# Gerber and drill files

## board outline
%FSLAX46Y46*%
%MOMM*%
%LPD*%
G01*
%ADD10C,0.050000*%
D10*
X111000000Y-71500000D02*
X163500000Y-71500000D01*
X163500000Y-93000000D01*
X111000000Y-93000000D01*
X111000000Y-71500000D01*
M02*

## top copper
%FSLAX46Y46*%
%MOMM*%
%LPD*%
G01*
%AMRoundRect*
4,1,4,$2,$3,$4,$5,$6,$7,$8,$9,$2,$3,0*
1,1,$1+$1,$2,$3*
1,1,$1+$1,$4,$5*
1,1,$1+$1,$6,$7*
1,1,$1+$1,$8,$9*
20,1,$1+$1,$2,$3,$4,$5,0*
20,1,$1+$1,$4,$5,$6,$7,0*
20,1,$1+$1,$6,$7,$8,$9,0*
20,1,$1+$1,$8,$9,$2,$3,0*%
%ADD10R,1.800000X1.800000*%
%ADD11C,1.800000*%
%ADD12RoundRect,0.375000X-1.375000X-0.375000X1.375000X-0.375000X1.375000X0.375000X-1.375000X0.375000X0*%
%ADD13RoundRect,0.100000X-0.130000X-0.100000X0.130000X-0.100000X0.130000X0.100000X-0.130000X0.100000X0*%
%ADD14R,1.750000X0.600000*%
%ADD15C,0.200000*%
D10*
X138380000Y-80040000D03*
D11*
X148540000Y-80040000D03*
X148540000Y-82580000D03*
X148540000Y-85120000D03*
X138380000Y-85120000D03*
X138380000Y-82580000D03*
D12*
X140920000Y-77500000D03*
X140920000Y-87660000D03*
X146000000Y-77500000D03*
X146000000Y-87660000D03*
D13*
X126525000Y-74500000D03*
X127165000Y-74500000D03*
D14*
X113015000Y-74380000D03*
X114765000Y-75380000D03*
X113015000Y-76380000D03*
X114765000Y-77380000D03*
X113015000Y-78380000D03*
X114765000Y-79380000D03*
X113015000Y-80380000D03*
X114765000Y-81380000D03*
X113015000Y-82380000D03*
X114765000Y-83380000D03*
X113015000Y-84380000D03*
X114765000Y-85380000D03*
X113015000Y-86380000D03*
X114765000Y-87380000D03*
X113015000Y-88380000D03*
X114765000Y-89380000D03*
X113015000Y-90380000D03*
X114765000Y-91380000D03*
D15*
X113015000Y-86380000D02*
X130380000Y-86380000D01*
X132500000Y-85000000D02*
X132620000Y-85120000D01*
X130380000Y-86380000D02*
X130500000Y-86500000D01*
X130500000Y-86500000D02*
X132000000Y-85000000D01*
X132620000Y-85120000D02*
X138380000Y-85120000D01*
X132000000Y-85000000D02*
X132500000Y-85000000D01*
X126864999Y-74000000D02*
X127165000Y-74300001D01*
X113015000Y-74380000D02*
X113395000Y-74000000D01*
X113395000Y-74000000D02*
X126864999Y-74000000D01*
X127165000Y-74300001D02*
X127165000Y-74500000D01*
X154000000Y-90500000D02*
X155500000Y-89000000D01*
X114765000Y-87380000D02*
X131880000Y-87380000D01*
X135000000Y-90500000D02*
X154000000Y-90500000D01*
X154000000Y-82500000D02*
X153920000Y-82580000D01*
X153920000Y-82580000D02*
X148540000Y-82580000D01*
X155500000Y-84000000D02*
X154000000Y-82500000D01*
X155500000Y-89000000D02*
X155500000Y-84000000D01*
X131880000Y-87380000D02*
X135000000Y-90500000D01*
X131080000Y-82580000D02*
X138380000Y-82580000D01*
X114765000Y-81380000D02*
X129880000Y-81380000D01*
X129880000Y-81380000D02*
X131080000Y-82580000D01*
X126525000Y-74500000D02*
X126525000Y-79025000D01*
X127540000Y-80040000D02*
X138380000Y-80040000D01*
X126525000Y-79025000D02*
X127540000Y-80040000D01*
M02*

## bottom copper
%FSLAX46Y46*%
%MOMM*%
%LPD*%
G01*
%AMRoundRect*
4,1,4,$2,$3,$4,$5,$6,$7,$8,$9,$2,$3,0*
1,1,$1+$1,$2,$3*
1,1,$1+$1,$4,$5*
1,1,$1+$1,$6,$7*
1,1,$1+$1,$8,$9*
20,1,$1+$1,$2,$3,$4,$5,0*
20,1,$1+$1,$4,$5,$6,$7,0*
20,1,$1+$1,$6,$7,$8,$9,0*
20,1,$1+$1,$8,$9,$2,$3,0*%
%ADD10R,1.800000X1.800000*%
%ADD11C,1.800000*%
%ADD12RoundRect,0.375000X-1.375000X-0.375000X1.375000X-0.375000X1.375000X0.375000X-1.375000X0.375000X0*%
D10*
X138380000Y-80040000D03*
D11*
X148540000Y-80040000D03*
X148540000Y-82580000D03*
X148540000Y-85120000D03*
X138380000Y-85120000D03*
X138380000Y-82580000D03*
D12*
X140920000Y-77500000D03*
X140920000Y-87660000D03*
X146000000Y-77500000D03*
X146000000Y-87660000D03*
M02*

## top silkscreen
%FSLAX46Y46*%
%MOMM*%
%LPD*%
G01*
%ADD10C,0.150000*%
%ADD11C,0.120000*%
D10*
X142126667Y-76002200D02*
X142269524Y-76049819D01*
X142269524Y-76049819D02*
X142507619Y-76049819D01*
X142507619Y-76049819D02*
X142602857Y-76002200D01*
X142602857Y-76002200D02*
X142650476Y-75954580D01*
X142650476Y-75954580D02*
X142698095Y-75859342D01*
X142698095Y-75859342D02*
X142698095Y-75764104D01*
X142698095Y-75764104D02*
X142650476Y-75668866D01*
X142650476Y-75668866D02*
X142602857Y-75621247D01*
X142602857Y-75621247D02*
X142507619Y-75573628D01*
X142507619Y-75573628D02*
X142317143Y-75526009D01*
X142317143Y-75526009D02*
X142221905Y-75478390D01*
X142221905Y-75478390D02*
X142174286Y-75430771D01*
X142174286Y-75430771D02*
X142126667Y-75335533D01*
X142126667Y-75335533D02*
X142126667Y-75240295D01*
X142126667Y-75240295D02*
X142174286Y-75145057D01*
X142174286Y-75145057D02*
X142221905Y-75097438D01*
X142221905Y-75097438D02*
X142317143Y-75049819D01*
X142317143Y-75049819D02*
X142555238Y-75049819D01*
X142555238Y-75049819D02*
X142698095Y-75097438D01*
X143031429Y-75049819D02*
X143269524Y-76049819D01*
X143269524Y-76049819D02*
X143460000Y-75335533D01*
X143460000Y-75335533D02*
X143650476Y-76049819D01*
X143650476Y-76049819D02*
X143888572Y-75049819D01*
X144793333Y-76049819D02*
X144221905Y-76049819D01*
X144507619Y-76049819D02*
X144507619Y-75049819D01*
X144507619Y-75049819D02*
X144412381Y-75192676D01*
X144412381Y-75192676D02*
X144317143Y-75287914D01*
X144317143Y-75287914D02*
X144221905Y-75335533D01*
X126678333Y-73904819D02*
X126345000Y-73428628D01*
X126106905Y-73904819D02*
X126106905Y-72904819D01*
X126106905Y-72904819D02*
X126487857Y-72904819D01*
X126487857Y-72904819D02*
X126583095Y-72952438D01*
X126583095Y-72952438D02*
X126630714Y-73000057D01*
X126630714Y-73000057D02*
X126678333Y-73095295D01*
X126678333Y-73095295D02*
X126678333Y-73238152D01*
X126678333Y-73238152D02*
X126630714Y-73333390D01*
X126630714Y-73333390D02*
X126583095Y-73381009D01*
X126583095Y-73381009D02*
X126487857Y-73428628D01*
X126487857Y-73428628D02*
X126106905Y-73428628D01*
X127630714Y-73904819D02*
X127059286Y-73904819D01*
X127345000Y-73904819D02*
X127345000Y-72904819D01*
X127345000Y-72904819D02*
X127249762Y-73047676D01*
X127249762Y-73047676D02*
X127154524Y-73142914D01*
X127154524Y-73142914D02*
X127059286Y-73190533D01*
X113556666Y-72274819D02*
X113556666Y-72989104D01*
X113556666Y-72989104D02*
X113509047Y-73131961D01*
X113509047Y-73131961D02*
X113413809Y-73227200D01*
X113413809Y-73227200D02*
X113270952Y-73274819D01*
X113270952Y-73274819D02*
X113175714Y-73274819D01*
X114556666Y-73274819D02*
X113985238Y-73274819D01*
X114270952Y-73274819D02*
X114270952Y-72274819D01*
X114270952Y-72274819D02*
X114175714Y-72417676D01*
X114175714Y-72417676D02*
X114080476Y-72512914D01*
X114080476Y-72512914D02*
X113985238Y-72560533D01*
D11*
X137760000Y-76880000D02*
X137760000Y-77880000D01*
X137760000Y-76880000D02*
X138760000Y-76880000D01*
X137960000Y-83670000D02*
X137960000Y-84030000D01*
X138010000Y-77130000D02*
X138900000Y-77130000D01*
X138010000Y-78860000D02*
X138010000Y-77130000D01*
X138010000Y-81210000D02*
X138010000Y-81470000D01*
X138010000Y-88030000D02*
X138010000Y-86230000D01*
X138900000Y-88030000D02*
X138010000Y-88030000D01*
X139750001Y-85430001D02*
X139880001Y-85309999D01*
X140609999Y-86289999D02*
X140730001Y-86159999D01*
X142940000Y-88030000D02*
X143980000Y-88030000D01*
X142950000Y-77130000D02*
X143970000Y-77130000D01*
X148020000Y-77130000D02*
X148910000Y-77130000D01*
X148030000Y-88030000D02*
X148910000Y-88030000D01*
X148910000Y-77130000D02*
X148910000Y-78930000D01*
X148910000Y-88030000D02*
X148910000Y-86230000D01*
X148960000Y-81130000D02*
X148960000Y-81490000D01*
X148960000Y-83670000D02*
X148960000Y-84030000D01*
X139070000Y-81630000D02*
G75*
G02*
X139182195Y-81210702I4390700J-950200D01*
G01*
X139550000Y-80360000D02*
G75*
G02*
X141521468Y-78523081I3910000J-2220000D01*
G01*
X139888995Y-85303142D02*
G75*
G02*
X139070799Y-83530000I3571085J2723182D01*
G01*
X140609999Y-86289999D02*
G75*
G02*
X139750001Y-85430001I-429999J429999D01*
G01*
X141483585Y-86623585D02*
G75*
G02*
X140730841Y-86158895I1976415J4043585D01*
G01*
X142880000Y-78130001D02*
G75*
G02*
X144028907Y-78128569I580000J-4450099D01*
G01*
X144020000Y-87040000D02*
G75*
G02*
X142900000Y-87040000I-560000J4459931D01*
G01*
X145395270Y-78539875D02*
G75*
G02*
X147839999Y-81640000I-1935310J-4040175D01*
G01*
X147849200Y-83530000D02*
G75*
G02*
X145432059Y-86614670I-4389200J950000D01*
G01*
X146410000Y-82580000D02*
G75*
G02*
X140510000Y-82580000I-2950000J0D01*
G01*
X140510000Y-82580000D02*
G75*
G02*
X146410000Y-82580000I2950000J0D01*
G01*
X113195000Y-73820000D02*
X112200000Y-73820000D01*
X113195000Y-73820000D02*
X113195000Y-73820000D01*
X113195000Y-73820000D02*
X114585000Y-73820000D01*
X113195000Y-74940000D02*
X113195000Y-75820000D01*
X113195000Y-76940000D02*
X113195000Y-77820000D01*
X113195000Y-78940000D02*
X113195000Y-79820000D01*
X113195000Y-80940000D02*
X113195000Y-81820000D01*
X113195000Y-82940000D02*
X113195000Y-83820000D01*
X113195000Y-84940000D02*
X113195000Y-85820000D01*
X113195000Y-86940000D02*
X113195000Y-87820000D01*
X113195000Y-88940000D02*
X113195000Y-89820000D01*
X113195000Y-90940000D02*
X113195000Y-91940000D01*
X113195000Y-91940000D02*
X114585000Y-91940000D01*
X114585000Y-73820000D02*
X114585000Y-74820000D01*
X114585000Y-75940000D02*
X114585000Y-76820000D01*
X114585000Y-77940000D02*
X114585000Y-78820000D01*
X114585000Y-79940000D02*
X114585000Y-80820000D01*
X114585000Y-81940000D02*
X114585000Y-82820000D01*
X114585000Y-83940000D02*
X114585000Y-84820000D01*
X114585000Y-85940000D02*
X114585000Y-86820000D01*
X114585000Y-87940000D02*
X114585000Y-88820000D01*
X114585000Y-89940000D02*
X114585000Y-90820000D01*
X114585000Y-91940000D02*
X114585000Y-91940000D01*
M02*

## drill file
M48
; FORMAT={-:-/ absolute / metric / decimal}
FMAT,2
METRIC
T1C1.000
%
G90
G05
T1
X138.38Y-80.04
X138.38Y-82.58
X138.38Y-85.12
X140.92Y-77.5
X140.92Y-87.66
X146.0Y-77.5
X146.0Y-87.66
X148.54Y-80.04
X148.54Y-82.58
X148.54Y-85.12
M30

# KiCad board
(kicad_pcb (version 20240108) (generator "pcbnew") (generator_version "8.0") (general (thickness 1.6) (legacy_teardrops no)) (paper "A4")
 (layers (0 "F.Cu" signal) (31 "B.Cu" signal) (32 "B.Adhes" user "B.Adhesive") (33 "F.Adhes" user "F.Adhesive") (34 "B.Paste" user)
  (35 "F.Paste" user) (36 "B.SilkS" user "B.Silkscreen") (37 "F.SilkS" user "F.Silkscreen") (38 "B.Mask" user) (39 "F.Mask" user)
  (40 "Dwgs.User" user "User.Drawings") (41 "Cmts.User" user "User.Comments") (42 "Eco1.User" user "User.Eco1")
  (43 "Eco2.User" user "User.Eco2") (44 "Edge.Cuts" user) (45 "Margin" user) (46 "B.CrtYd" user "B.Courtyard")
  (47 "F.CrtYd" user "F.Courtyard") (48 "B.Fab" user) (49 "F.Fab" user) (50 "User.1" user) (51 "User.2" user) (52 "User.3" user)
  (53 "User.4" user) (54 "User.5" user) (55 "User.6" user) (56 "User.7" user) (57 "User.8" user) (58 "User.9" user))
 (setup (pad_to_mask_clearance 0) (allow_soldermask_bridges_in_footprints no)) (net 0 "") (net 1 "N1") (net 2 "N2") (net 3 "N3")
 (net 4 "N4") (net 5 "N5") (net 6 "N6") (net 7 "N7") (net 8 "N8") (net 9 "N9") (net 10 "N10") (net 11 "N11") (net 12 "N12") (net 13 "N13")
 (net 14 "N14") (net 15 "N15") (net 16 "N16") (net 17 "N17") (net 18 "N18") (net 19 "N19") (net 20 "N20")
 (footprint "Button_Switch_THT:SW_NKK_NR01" (layer "F.Cu") (at 138.38 80.04)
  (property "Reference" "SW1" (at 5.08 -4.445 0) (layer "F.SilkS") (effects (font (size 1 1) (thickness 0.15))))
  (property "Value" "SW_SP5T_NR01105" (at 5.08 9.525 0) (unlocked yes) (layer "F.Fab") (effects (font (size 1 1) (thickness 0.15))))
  (fp_line (start -0.62 -3.16) (end -0.62 -2.16) (stroke (width 0.12) (type default)) (layer "F.SilkS"))
  (fp_line (start -0.62 -3.16) (end 0.38 -3.16) (stroke (width 0.12) (type default)) (layer "F.SilkS"))
  (fp_line (start -0.42 3.63) (end -0.42 3.99) (stroke (width 0.12) (type default)) (layer "F.SilkS"))
  (fp_line (start -0.37 -2.91) (end 0.52 -2.91) (stroke (width 0.12) (type default)) (layer "F.SilkS"))
  (fp_line (start -0.37 -1.18) (end -0.37 -2.91) (stroke (width 0.12) (type default)) (layer "F.SilkS"))
  (fp_line (start -0.37 1.17) (end -0.37 1.43) (stroke (width 0.12) (type default)) (layer "F.SilkS"))
  (fp_line (start -0.37 7.99) (end -0.37 6.19) (stroke (width 0.12) (type default)) (layer "F.SilkS"))
  (fp_line (start 0.52 7.99) (end -0.37 7.99) (stroke (width 0.12) (type default)) (layer "F.SilkS"))
  (fp_line (start 1.370001 5.390001) (end 1.500001 5.269999) (stroke (width 0.12) (type default)) (layer "F.SilkS"))
  (fp_line (start 2.229999 6.249999) (end 2.350001 6.119999) (stroke (width 0.12) (type default)) (layer "F.SilkS"))
  (fp_line (start 4.56 7.99) (end 5.6 7.99) (stroke (width 0.12) (type default)) (layer "F.SilkS"))
  (fp_line (start 4.57 -2.91) (end 5.59 -2.91) (stroke (width 0.12) (type default)) (layer "F.SilkS"))
  (fp_line (start 9.64 -2.91) (end 10.53 -2.91) (stroke (width 0.12) (type default)) (layer "F.SilkS"))
  (fp_line (start 9.65 7.99) (end 10.53 7.99) (stroke (width 0.12) (type default)) (layer "F.SilkS"))
  (fp_line (start 10.53 -2.91) (end 10.53 -1.11) (stroke (width 0.12) (type default)) (layer "F.SilkS"))
  (fp_line (start 10.53 7.99) (end 10.53 6.19) (stroke (width 0.12) (type default)) (layer "F.SilkS"))
  (fp_line (start 10.58 1.09) (end 10.58 1.45) (stroke (width 0.12) (type default)) (layer "F.SilkS"))
  (fp_line (start 10.58 3.63) (end 10.58 3.99) (stroke (width 0.12) (type default)) (layer "F.SilkS"))
  (fp_arc (start 0.69 1.59) (mid 0.74103 1.378995) (end 0.802194 1.170702) (stroke (width 0.12) (type default)) (layer "F.SilkS"))
  (fp_arc (start 1.17 0.32) (mid 2.01489 -0.74962) (end 3.141468 -1.516919) (stroke (width 0.12) (type default)) (layer "F.SilkS"))
  (fp_arc (start 1.508995 5.263142) (mid 1.002352 4.421582) (end 0.690799 3.49) (stroke (width 0.12) (type default)) (layer "F.SilkS"))
  (fp_arc (start 2.229999 6.249999) (mid 1.370001 6.249999) (end 1.370001 5.390001) (stroke (width 0.12) (type default)) (layer "F.SilkS"))
  (fp_arc (start 3.103585 6.583585) (mid 2.715769 6.369779) (end 2.350841 6.118895) (stroke (width 0.12) (type default)) (layer "F.SilkS"))
  (fp_arc (start 4.5 -1.909999) (mid 5.074407 -1.947633) (end 5.648907 -1.911431) (stroke (width 0.12) (type default)) (layer "F.SilkS"))
  (fp_arc (start 5.64 7) (mid 5.08 7.03502) (end 4.52 7) (stroke (width 0.12) (type default)) (layer "F.SilkS"))
  (fp_arc (start 7.01527 -1.500125) (mid 8.597573 -0.233907) (end 9.459999 1.6) (stroke (width 0.12) (type default)) (layer "F.SilkS"))
  (fp_arc (start 9.4692 3.49) (mid 8.614855 5.309905) (end 7.052059 6.574669) (stroke (width 0.12) (type default)) (layer "F.SilkS"))
  (fp_circle (center 5.08 2.54) (end 8.03 2.54) (stroke (width 0.12) (type default)) (fill none) (layer "F.SilkS"))
  (pad "1" thru_hole rect (at 0 0) (size 1.8 1.8) (drill 1) (layers "*.Cu" "*.Mask") (remove_unused_layers no) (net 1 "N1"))
  (pad "2" thru_hole circle (at 10.16 0) (size 1.8 1.8) (drill 1) (layers "*.Cu" "*.Mask") (remove_unused_layers no) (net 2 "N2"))
  (pad "3" thru_hole circle (at 10.16 2.54) (size 1.8 1.8) (drill 1) (layers "*.Cu" "*.Mask") (remove_unused_layers no) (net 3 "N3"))
  (pad "4" thru_hole circle (at 10.16 5.08) (size 1.8 1.8) (drill 1) (layers "*.Cu" "*.Mask") (remove_unused_layers no) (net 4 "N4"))
  (pad "5" thru_hole circle (at 0 5.08) (size 1.8 1.8) (drill 1) (layers "*.Cu" "*.Mask") (remove_unused_layers no) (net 4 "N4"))
  (pad "C" thru_hole circle (at 0 2.54) (size 1.8 1.8) (drill 1) (layers "*.Cu" "*.Mask") (remove_unused_layers no) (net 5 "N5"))
  (pad "MP" thru_hole roundrect (at 2.54 -2.54) (size 3.5 1.5) (drill 1) (layers "*.Cu" "*.Mask") (remove_unused_layers no)
   (roundrect_rratio 0.25) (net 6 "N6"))
  (pad "MP" thru_hole roundrect (at 2.54 7.62) (size 3.5 1.5) (drill 1) (layers "*.Cu" "*.Mask") (remove_unused_layers no)
   (roundrect_rratio 0.25) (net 6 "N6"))
  (pad "MP" thru_hole roundrect (at 7.62 -2.54) (size 3.5 1.5) (drill 1) (layers "*.Cu" "*.Mask") (remove_unused_layers no)
   (roundrect_rratio 0.25) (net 6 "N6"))
  (pad "MP" thru_hole roundrect (at 7.62 7.62) (size 3.5 1.5) (drill 1) (layers "*.Cu" "*.Mask") (remove_unused_layers no)
   (roundrect_rratio 0.25) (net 6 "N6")))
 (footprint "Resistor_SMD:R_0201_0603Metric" (layer "F.Cu") (at 126.845 74.5)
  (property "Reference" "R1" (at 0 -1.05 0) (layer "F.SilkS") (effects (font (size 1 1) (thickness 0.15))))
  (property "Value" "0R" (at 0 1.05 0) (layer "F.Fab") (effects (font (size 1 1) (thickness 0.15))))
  (pad "" smd roundrect (at -0.345 0) (size 0.318 0.36) (layers "F.Paste") (roundrect_rratio 0.25))
  (pad "" smd roundrect (at 0.345 0) (size 0.318 0.36) (layers "F.Paste") (roundrect_rratio 0.25))
  (pad "1" smd roundrect (at -0.32 0) (size 0.46 0.4) (layers "F.Cu" "F.Mask") (roundrect_rratio 0.25) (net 1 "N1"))
  (pad "2" smd roundrect (at 0.32 0) (size 0.46 0.4) (layers "F.Cu" "F.Mask") (roundrect_rratio 0.25) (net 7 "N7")))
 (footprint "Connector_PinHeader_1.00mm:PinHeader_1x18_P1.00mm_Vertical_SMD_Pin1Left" (layer "F.Cu") (at 113.89 82.88)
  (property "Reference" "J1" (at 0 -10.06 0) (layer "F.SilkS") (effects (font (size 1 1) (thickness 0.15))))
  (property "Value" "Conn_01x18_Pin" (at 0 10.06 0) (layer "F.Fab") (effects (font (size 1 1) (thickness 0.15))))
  (fp_line (start -0.695 -9.06) (end -1.69 -9.06) (stroke (width 0.12) (type solid)) (layer "F.SilkS"))
  (fp_line (start -0.695 -9.06) (end -0.695 -9.06) (stroke (width 0.12) (type solid)) (layer "F.SilkS"))
  (fp_line (start -0.695 -9.06) (end 0.695 -9.06) (stroke (width 0.12) (type solid)) (layer "F.SilkS"))
  (fp_line (start -0.695 -7.94) (end -0.695 -7.06) (stroke (width 0.12) (type solid)) (layer "F.SilkS"))
  (fp_line (start -0.695 -5.94) (end -0.695 -5.06) (stroke (width 0.12) (type solid)) (layer "F.SilkS"))
  (fp_line (start -0.695 -3.94) (end -0.695 -3.06) (stroke (width 0.12) (type solid)) (layer "F.SilkS"))
  (fp_line (start -0.695 -1.94) (end -0.695 -1.06) (stroke (width 0.12) (type solid)) (layer "F.SilkS"))
  (fp_line (start -0.695 0.06) (end -0.695 0.94) (stroke (width 0.12) (type solid)) (layer "F.SilkS"))
  (fp_line (start -0.695 2.06) (end -0.695 2.94) (stroke (width 0.12) (type solid)) (layer "F.SilkS"))
  (fp_line (start -0.695 4.06) (end -0.695 4.94) (stroke (width 0.12) (type solid)) (layer "F.SilkS"))
  (fp_line (start -0.695 6.06) (end -0.695 6.94) (stroke (width 0.12) (type solid)) (layer "F.SilkS"))
  (fp_line (start -0.695 8.06) (end -0.695 9.06) (stroke (width 0.12) (type solid)) (layer "F.SilkS"))
  (fp_line (start -0.695 9.06) (end 0.695 9.06) (stroke (width 0.12) (type solid)) (layer "F.SilkS"))
  (fp_line (start 0.695 -9.06) (end 0.695 -8.06) (stroke (width 0.12) (type solid)) (layer "F.SilkS"))
  (fp_line (start 0.695 -6.94) (end 0.695 -6.06) (stroke (width 0.12) (type solid)) (layer "F.SilkS"))
  (fp_line (start 0.695 -4.94) (end 0.695 -4.06) (stroke (width 0.12) (type solid)) (layer "F.SilkS"))
  (fp_line (start 0.695 -2.94) (end 0.695 -2.06) (stroke (width 0.12) (type solid)) (layer "F.SilkS"))
  (fp_line (start 0.695 -0.94) (end 0.695 -0.06) (stroke (width 0.12) (type solid)) (layer "F.SilkS"))
  (fp_line (start 0.695 1.06) (end 0.695 1.94) (stroke (width 0.12) (type solid)) (layer "F.SilkS"))
  (fp_line (start 0.695 3.06) (end 0.695 3.94) (stroke (width 0.12) (type solid)) (layer "F.SilkS"))
  (fp_line (start 0.695 5.06) (end 0.695 5.94) (stroke (width 0.12) (type solid)) (layer "F.SilkS"))
  (fp_line (start 0.695 7.06) (end 0.695 7.94) (stroke (width 0.12) (type solid)) (layer "F.SilkS"))
  (fp_line (start 0.695 9.06) (end 0.695 9.06) (stroke (width 0.12) (type solid)) (layer "F.SilkS"))
  (pad "1" smd rect (at -0.875 -8.5) (size 1.75 0.6) (layers "F.Cu" "F.Paste" "F.Mask") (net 7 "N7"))
  (pad "2" smd rect (at 0.875 -7.5) (size 1.75 0.6) (layers "F.Cu" "F.Paste" "F.Mask") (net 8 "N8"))
  (pad "3" smd rect (at -0.875 -6.5) (size 1.75 0.6) (layers "F.Cu" "F.Paste" "F.Mask") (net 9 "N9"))
  (pad "4" smd rect (at 0.875 -5.5) (size 1.75 0.6) (layers "F.Cu" "F.Paste" "F.Mask") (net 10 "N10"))
  (pad "5" smd rect (at -0.875 -4.5) (size 1.75 0.6) (layers "F.Cu" "F.Paste" "F.Mask") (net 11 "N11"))
  (pad "6" smd rect (at 0.875 -3.5) (size 1.75 0.6) (layers "F.Cu" "F.Paste" "F.Mask") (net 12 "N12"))
  (pad "7" smd rect (at -0.875 -2.5) (size 1.75 0.6) (layers "F.Cu" "F.Paste" "F.Mask") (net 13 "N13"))
  (pad "8" smd rect (at 0.875 -1.5) (size 1.75 0.6) (layers "F.Cu" "F.Paste" "F.Mask") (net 5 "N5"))
  (pad "9" smd rect (at -0.875 -0.5) (size 1.75 0.6) (layers "F.Cu" "F.Paste" "F.Mask") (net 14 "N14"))
  (pad "10" smd rect (at 0.875 0.5) (size 1.75 0.6) (layers "F.Cu" "F.Paste" "F.Mask") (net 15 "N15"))
  (pad "11" smd rect (at -0.875 1.5) (size 1.75 0.6) (layers "F.Cu" "F.Paste" "F.Mask") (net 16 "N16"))
  (pad "12" smd rect (at 0.875 2.5) (size 1.75 0.6) (layers "F.Cu" "F.Paste" "F.Mask") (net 4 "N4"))
  (pad "13" smd rect (at -0.875 3.5) (size 1.75 0.6) (layers "F.Cu" "F.Paste" "F.Mask") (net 4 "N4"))
  (pad "14" smd rect (at 0.875 4.5) (size 1.75 0.6) (layers "F.Cu" "F.Paste" "F.Mask") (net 3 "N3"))
  (pad "15" smd rect (at -0.875 5.5) (size 1.75 0.6) (layers "F.Cu" "F.Paste" "F.Mask") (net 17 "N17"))
  (pad "16" smd rect (at 0.875 6.5) (size 1.75 0.6) (layers "F.Cu" "F.Paste" "F.Mask") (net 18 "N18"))
  (pad "17" smd rect (at -0.875 7.5) (size 1.75 0.6) (layers "F.Cu" "F.Paste" "F.Mask") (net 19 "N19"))
  (pad "18" smd rect (at 0.875 8.5) (size 1.75 0.6) (layers "F.Cu" "F.Paste" "F.Mask") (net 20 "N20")))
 (gr_rect (start 111 71.5) (end 163.5 93) (stroke (width 0.05) (type default)) (fill none) (layer "Edge.Cuts"))
 (segment (start 113.015 86.38) (end 130.38 86.38) (width 0.2) (layer "F.Cu") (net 4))
 (segment (start 132.5 85) (end 132.62 85.12) (width 0.2) (layer "F.Cu") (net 4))
 (segment (start 130.38 86.38) (end 130.5 86.5) (width 0.2) (layer "F.Cu") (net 4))
 (segment (start 130.5 86.5) (end 132 85) (width 0.2) (layer "F.Cu") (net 4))
 (segment (start 132.62 85.12) (end 138.38 85.12) (width 0.2) (layer "F.Cu") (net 4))
 (segment (start 132 85) (end 132.5 85) (width 0.2) (layer "F.Cu") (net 4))
 (segment (start 126.864999 74) (end 127.165 74.300001) (width 0.2) (layer "F.Cu") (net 7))
 (segment (start 113.015 74.38) (end 113.395 74) (width 0.2) (layer "F.Cu") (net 7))
 (segment (start 113.395 74) (end 126.864999 74) (width 0.2) (layer "F.Cu") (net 7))
 (segment (start 127.165 74.300001) (end 127.165 74.5) (width 0.2) (layer "F.Cu") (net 7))
 (segment (start 154 90.5) (end 155.5 89) (width 0.2) (layer "F.Cu") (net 3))
 (segment (start 114.765 87.38) (end 131.88 87.38) (width 0.2) (layer "F.Cu") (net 3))
 (segment (start 135 90.5) (end 154 90.5) (width 0.2) (layer "F.Cu") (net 3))
 (segment (start 154 82.5) (end 153.92 82.58) (width 0.2) (layer "F.Cu") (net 3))
 (segment (start 153.92 82.58) (end 148.54 82.58) (width 0.2) (layer "F.Cu") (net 3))
 (segment (start 155.5 84) (end 154 82.5) (width 0.2) (layer "F.Cu") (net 3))
 (segment (start 155.5 89) (end 155.5 84) (width 0.2) (layer "F.Cu") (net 3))
 (segment (start 131.88 87.38) (end 135 90.5) (width 0.2) (layer "F.Cu") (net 3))
 (segment (start 131.08 82.58) (end 138.38 82.58) (width 0.2) (layer "F.Cu") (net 5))
 (segment (start 114.765 81.38) (end 129.88 81.38) (width 0.2) (layer "F.Cu") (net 5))
 (segment (start 129.88 81.38) (end 131.08 82.58) (width 0.2) (layer "F.Cu") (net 5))
 (segment (start 126.525 74.5) (end 126.525 79.025) (width 0.2) (layer "F.Cu") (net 1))
 (segment (start 127.54 80.04) (end 138.38 80.04) (width 0.2) (layer "F.Cu") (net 1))
 (segment (start 126.525 79.025) (end 127.54 80.04) (width 0.2) (layer "F.Cu") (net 1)))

